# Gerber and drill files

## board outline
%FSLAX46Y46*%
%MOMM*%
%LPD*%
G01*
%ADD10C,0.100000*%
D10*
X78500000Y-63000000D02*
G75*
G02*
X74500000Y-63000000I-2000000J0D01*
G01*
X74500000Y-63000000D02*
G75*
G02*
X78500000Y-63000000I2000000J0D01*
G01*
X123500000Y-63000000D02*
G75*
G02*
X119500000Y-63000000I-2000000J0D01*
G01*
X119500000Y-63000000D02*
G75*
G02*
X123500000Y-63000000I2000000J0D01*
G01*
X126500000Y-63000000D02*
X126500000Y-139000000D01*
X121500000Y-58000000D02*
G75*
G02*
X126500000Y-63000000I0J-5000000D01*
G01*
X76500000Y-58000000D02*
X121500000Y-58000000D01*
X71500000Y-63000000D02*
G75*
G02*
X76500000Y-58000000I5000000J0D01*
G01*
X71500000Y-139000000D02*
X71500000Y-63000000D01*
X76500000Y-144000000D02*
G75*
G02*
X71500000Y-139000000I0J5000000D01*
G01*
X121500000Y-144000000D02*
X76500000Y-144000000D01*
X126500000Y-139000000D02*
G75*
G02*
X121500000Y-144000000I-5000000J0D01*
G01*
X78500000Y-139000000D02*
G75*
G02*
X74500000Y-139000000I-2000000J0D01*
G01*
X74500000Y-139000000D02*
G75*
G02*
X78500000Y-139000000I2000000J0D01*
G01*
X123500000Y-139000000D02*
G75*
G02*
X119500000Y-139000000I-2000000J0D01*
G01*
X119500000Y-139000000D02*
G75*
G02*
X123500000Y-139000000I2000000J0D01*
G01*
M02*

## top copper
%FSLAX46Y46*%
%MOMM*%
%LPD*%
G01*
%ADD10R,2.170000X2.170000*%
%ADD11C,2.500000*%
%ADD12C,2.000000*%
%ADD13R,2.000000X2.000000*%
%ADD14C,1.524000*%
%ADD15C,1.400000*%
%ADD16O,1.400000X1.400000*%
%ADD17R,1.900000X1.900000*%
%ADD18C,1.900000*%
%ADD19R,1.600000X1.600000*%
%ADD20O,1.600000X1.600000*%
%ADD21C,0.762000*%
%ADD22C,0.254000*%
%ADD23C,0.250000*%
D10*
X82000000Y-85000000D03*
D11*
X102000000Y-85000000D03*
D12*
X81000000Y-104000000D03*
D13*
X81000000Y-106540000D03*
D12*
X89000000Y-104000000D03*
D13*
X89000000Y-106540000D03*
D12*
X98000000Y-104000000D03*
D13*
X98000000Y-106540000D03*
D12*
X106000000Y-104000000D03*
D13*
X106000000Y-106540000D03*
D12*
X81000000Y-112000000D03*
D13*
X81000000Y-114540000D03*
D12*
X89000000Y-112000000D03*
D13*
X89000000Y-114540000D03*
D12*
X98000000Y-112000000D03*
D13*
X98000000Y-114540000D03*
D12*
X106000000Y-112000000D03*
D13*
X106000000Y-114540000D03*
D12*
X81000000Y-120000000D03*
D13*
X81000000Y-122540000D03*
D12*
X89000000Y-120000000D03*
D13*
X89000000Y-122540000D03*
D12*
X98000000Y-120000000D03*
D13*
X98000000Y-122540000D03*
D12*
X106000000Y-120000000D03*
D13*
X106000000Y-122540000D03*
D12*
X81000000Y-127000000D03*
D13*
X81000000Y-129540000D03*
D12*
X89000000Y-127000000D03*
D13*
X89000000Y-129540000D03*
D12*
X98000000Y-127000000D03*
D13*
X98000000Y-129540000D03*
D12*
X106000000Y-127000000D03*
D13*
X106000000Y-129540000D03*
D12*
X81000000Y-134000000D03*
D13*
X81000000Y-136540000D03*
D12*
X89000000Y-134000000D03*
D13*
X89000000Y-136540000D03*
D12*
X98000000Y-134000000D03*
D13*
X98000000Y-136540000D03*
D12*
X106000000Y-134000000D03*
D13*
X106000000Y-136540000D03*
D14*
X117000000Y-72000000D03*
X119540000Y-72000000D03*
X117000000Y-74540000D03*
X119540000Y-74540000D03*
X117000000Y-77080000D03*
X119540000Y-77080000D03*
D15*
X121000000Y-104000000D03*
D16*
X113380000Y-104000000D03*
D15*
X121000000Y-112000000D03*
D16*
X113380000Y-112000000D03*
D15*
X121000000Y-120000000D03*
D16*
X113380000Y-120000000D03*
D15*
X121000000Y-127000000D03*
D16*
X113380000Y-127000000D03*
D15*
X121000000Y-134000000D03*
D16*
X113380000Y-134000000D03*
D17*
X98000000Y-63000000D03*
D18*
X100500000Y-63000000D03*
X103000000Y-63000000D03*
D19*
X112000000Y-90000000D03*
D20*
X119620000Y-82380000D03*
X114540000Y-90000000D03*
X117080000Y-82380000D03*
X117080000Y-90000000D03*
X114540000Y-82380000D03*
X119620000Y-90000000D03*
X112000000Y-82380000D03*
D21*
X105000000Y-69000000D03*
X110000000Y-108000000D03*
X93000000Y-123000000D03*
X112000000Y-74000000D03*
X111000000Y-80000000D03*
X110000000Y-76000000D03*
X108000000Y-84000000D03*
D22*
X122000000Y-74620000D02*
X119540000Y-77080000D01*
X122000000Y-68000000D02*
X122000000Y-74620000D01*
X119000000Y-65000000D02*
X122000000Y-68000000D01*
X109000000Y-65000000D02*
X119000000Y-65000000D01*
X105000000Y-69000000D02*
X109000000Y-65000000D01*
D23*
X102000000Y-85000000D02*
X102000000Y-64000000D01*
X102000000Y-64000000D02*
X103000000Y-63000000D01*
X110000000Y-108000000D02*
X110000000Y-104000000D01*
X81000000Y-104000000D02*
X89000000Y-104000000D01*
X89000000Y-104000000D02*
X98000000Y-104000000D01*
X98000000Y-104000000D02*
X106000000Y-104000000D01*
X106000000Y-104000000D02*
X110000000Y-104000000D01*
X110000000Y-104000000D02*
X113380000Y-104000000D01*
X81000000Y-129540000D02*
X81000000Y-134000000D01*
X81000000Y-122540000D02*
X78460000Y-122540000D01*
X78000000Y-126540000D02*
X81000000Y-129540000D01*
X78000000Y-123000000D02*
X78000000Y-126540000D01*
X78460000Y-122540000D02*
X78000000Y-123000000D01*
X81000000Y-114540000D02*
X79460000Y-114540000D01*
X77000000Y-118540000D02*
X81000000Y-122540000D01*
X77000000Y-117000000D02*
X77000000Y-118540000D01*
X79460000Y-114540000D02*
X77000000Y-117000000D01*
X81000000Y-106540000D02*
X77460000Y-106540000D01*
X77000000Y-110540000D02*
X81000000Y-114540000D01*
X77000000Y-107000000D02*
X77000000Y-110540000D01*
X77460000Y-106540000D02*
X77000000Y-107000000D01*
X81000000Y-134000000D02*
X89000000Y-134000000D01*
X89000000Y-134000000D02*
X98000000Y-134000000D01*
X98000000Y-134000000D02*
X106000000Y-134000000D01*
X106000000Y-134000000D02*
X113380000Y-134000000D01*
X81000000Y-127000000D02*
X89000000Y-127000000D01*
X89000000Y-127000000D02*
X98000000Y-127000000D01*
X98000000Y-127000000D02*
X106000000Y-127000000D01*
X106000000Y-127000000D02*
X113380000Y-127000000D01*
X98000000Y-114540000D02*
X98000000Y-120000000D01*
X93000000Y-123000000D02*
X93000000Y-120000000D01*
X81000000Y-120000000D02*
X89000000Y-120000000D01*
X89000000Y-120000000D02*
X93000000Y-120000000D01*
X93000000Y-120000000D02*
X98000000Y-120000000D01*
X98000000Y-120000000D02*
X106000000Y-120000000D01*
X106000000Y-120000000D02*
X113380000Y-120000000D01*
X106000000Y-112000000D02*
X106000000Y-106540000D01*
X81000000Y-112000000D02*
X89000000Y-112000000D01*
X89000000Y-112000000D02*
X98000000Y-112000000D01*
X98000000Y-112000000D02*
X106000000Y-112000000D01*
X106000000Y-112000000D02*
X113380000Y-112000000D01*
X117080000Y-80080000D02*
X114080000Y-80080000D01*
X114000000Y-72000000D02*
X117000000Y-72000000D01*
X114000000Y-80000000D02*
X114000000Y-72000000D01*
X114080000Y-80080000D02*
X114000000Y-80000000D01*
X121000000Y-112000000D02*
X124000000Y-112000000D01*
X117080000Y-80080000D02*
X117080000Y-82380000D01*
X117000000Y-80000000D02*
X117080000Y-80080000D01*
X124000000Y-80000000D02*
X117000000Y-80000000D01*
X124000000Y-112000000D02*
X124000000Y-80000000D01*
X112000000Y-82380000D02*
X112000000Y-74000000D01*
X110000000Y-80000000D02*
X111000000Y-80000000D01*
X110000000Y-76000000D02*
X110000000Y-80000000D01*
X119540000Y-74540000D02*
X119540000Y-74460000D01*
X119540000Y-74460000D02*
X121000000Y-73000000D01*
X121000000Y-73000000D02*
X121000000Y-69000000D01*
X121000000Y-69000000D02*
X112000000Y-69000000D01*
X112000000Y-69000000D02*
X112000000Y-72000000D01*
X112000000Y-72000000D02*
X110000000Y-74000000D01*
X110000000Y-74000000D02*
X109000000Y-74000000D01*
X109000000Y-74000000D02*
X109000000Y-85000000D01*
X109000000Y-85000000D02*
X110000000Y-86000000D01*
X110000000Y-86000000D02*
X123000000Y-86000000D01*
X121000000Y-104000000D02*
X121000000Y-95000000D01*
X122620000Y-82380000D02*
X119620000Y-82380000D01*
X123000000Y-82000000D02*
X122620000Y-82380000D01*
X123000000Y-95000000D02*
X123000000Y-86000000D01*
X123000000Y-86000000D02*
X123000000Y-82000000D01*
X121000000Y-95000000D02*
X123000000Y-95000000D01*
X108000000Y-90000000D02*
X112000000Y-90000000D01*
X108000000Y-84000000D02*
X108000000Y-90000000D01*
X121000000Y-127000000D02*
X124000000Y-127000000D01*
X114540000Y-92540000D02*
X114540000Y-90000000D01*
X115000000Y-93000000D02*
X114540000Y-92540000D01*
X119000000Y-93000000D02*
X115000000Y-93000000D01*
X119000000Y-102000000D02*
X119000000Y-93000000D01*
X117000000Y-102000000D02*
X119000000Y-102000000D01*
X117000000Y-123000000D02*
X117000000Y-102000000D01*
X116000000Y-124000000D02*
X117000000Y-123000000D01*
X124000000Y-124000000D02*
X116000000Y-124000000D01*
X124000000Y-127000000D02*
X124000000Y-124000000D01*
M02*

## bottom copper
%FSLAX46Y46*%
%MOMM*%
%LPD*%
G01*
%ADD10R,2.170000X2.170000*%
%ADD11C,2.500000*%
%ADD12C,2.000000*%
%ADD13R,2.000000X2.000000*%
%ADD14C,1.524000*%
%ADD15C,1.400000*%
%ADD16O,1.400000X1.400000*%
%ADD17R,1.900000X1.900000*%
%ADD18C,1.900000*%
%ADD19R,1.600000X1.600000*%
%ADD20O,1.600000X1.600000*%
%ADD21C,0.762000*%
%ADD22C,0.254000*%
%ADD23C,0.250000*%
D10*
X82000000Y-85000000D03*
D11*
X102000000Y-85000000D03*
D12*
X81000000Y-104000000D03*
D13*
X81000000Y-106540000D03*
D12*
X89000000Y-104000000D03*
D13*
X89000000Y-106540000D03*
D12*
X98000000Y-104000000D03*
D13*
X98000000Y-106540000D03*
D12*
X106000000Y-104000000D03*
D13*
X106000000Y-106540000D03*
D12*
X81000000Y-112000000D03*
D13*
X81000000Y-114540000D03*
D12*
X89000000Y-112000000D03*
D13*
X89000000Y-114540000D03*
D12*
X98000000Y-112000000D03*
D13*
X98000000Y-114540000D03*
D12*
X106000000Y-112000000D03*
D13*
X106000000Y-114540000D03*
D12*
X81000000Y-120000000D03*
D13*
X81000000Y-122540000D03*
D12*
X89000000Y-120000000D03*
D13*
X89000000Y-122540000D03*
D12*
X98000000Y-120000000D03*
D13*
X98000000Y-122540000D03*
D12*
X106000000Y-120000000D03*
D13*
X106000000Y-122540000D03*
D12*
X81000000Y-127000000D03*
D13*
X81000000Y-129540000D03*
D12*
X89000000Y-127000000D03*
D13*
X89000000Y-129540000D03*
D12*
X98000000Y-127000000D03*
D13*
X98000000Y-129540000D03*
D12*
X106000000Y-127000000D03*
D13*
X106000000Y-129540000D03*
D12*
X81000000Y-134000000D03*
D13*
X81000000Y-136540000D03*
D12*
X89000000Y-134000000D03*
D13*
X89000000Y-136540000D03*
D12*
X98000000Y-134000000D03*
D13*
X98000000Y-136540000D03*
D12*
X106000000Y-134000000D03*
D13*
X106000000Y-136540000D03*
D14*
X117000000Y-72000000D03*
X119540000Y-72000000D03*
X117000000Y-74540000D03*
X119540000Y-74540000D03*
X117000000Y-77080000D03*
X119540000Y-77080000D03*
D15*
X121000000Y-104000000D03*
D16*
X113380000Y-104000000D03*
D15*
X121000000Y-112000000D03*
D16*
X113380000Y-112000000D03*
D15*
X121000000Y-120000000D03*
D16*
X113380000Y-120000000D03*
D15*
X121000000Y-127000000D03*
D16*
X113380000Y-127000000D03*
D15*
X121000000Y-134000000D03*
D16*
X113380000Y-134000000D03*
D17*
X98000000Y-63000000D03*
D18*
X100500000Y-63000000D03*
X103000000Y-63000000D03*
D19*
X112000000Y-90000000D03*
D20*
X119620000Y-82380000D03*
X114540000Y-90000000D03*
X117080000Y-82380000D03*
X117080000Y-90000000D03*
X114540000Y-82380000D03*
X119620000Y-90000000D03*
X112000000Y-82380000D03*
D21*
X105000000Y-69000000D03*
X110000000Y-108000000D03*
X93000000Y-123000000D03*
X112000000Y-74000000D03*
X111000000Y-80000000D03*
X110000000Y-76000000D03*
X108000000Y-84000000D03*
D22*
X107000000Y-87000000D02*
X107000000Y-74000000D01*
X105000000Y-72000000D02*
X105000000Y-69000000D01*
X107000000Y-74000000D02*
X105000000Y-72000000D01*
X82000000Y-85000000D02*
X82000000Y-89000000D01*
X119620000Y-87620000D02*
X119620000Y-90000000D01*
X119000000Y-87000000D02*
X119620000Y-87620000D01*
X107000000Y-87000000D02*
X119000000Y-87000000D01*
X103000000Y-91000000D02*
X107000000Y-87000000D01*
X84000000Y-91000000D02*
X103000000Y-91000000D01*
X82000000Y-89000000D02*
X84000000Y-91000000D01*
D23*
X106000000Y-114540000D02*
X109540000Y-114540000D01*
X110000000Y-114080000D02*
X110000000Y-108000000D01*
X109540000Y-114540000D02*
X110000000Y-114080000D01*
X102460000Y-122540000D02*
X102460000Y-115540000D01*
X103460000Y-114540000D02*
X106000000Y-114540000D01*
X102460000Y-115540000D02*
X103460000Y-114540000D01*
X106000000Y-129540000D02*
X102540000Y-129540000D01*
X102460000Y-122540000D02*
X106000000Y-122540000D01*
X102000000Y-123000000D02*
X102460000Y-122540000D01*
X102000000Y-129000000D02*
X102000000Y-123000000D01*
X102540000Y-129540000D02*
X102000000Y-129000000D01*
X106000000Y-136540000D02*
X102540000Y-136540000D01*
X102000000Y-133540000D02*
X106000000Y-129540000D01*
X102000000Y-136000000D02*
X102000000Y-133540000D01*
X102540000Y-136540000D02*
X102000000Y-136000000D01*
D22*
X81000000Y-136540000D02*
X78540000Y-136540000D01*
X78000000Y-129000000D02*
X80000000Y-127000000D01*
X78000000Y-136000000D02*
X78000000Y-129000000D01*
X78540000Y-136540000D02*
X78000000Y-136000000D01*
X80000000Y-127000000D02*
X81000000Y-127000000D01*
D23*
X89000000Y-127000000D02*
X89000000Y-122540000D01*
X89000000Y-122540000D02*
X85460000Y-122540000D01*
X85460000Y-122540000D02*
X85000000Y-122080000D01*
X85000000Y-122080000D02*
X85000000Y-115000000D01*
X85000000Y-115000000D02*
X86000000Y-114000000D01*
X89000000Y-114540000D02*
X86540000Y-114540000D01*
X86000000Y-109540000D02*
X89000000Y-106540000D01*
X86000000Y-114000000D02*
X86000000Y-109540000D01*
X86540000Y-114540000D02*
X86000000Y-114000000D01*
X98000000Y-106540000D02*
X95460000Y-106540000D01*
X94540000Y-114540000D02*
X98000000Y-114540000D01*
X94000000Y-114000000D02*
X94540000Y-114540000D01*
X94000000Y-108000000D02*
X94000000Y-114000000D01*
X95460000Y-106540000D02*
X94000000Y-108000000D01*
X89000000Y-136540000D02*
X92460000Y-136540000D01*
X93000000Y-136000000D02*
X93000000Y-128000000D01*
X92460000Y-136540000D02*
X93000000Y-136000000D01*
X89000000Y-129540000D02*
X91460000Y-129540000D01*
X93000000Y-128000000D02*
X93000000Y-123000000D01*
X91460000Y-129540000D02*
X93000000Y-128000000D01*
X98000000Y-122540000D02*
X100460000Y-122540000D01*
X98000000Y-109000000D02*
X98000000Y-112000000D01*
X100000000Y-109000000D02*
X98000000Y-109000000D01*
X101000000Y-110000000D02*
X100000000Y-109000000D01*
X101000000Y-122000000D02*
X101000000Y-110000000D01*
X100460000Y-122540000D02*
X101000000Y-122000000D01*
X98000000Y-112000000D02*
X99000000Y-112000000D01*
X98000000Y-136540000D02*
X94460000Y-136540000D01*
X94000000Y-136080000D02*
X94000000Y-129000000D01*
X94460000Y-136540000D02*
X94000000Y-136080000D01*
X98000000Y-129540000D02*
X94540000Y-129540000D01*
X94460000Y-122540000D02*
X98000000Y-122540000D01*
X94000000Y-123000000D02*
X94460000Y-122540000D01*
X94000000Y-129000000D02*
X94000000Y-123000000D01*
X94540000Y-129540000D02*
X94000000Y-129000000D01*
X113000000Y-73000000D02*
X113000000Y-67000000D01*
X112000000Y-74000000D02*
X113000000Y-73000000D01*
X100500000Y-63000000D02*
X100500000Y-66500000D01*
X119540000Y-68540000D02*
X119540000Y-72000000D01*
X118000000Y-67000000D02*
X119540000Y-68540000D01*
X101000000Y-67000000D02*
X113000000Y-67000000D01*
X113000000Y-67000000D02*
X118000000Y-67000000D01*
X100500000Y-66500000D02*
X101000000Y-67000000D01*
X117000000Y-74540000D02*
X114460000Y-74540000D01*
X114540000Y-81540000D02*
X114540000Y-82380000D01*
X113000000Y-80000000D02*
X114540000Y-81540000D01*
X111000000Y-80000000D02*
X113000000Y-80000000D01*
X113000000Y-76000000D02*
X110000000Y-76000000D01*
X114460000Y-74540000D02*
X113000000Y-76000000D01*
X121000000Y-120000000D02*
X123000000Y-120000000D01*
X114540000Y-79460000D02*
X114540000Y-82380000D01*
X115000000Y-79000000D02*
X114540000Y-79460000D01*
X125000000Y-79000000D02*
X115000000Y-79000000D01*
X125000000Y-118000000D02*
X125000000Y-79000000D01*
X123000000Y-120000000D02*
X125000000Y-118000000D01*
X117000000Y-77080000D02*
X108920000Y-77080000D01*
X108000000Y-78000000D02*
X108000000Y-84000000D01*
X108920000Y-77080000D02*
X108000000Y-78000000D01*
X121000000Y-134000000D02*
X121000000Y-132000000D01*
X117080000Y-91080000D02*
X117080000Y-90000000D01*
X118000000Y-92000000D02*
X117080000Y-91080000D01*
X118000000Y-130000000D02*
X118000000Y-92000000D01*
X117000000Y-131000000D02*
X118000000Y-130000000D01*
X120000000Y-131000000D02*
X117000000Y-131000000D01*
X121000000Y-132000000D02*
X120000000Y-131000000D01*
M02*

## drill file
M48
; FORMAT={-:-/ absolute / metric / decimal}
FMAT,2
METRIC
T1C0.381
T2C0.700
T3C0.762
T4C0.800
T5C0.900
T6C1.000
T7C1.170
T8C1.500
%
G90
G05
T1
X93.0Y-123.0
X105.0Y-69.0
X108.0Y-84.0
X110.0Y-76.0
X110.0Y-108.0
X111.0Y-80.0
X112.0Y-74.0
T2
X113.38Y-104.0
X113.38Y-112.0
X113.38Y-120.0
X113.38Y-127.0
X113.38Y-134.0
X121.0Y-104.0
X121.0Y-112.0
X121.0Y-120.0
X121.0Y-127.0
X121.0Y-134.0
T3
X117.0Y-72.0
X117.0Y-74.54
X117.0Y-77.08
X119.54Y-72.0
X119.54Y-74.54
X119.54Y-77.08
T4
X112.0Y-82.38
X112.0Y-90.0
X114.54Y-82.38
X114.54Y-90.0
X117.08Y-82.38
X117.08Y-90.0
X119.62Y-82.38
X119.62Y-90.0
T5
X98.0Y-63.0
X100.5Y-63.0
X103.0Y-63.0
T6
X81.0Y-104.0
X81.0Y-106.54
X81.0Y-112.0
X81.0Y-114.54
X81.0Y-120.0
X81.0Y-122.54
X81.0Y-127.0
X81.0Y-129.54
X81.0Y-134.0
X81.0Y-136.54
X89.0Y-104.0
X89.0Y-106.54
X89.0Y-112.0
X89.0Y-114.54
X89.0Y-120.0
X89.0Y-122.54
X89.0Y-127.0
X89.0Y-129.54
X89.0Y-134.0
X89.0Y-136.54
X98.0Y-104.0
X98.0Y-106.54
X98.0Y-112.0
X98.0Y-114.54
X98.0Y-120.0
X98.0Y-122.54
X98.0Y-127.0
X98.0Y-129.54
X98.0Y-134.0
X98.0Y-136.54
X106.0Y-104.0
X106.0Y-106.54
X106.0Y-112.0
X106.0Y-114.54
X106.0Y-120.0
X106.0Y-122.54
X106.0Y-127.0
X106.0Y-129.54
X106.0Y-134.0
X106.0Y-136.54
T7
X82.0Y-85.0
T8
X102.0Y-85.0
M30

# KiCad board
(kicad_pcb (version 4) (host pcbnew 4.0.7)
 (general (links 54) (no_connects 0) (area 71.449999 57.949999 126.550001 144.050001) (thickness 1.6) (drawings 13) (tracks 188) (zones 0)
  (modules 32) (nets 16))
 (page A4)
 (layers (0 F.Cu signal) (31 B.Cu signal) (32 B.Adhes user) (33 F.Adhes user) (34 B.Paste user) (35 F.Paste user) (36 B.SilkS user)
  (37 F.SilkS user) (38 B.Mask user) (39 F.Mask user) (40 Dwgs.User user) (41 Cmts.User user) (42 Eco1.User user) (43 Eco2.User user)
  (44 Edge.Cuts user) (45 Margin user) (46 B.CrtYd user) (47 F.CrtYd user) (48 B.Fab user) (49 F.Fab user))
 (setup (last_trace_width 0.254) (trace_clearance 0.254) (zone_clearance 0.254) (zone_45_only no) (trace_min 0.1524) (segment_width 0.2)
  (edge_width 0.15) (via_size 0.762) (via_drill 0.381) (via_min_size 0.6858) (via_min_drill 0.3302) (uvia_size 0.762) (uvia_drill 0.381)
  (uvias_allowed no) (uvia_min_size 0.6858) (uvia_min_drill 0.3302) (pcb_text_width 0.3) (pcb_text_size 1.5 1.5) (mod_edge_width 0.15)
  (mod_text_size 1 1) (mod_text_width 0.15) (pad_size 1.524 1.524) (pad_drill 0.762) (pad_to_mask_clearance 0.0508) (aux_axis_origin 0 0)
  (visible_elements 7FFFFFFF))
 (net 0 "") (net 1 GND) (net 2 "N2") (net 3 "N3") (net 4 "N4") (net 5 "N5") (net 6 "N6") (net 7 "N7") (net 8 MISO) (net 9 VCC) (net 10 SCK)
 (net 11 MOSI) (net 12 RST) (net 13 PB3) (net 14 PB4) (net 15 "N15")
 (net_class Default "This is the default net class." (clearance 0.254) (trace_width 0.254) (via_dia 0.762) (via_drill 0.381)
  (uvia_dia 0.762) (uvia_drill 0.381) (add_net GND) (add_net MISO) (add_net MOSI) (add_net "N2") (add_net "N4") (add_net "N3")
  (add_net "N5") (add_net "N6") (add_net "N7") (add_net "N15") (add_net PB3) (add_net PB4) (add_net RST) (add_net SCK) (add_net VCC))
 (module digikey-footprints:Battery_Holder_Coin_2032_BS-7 (layer F.Cu) (at 82 85)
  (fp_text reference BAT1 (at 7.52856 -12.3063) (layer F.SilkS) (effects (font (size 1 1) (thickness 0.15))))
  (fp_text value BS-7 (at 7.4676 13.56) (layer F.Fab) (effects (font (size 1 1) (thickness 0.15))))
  (pad Neg thru_hole rect (at 0 0) (size 2.17 2.17) (drill 1.17) (layers *.Cu *.Mask) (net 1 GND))
  (pad Pos thru_hole circle (at 20 0) (size 2.5 2.5) (drill 1.5) (layers *.Cu *.Mask) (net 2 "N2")))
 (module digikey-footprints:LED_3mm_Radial (layer F.Cu) (at 81 104 90)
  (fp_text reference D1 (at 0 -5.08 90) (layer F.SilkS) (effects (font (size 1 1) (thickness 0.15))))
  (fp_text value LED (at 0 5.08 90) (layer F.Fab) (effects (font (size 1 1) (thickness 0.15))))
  (pad 2 thru_hole circle (at 0 0 90) (size 2 2) (drill 1) (layers *.Cu *.Mask) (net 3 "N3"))
  (pad 1 thru_hole rect (at -2.54 0 90) (size 2 2) (drill 1) (layers *.Cu *.Mask) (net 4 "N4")))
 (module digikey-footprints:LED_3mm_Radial (layer F.Cu) (at 89 104 90)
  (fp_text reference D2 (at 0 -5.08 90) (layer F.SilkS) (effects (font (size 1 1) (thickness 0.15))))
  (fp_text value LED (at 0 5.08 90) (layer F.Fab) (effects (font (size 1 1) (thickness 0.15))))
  (pad 2 thru_hole circle (at 0 0 90) (size 2 2) (drill 1) (layers *.Cu *.Mask) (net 3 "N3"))
  (pad 1 thru_hole rect (at -2.54 0 90) (size 2 2) (drill 1) (layers *.Cu *.Mask) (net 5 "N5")))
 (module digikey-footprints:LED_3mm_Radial (layer F.Cu) (at 98 104 90)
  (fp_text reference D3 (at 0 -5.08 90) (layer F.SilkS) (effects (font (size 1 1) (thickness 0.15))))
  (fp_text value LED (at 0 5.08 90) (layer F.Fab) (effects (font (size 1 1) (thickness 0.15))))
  (pad 2 thru_hole circle (at 0 0 90) (size 2 2) (drill 1) (layers *.Cu *.Mask) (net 3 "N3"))
  (pad 1 thru_hole rect (at -2.54 0 90) (size 2 2) (drill 1) (layers *.Cu *.Mask) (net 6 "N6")))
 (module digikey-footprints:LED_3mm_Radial (layer F.Cu) (at 106 104 90)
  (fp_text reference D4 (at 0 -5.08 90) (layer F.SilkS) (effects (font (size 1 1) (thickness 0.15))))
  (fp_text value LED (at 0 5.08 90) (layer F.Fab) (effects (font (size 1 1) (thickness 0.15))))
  (pad 2 thru_hole circle (at 0 0 90) (size 2 2) (drill 1) (layers *.Cu *.Mask) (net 3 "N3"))
  (pad 1 thru_hole rect (at -2.54 0 90) (size 2 2) (drill 1) (layers *.Cu *.Mask) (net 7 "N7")))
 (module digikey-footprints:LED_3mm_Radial (layer F.Cu) (at 81 112 90)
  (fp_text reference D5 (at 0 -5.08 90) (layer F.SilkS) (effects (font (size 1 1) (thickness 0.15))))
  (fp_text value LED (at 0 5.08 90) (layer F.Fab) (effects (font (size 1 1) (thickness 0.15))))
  (pad 2 thru_hole circle (at 0 0 90) (size 2 2) (drill 1) (layers *.Cu *.Mask) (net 7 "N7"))
  (pad 1 thru_hole rect (at -2.54 0 90) (size 2 2) (drill 1) (layers *.Cu *.Mask) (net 4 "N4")))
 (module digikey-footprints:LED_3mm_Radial (layer F.Cu) (at 89 112 90)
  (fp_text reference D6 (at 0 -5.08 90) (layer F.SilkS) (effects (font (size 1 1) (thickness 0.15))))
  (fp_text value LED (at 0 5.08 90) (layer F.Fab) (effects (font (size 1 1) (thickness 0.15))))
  (pad 2 thru_hole circle (at 0 0 90) (size 2 2) (drill 1) (layers *.Cu *.Mask) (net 7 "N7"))
  (pad 1 thru_hole rect (at -2.54 0 90) (size 2 2) (drill 1) (layers *.Cu *.Mask) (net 5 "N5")))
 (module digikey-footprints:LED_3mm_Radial (layer F.Cu) (at 98 112 90)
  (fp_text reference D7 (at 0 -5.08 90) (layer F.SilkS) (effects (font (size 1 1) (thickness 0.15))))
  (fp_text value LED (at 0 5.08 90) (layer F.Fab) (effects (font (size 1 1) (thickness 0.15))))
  (pad 2 thru_hole circle (at 0 0 90) (size 2 2) (drill 1) (layers *.Cu *.Mask) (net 7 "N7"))
  (pad 1 thru_hole rect (at -2.54 0 90) (size 2 2) (drill 1) (layers *.Cu *.Mask) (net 6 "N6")))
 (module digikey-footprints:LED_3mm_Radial (layer F.Cu) (at 106 112 90)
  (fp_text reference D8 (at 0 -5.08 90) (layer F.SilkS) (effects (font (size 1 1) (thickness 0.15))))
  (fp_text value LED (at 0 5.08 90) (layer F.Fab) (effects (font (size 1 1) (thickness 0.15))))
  (pad 2 thru_hole circle (at 0 0 90) (size 2 2) (drill 1) (layers *.Cu *.Mask) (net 7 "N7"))
  (pad 1 thru_hole rect (at -2.54 0 90) (size 2 2) (drill 1) (layers *.Cu *.Mask) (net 3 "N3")))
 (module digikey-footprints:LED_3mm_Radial (layer F.Cu) (at 81 120 90)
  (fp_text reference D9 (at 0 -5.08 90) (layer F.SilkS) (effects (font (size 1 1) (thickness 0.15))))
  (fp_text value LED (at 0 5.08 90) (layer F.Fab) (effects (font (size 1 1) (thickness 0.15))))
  (pad 2 thru_hole circle (at 0 0 90) (size 2 2) (drill 1) (layers *.Cu *.Mask) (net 6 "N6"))
  (pad 1 thru_hole rect (at -2.54 0 90) (size 2 2) (drill 1) (layers *.Cu *.Mask) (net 4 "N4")))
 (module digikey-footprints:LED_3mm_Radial (layer F.Cu) (at 89 120 90)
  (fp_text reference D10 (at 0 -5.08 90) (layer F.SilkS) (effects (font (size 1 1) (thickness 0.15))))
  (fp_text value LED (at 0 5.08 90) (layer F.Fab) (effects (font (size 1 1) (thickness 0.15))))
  (pad 2 thru_hole circle (at 0 0 90) (size 2 2) (drill 1) (layers *.Cu *.Mask) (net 6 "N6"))
  (pad 1 thru_hole rect (at -2.54 0 90) (size 2 2) (drill 1) (layers *.Cu *.Mask) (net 5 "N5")))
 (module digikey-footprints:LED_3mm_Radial (layer F.Cu) (at 98 120 90)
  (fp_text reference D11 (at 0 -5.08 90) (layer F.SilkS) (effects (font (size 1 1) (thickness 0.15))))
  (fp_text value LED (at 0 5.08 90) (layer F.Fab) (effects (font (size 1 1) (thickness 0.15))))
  (pad 2 thru_hole circle (at 0 0 90) (size 2 2) (drill 1) (layers *.Cu *.Mask) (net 6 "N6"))
  (pad 1 thru_hole rect (at -2.54 0 90) (size 2 2) (drill 1) (layers *.Cu *.Mask) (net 7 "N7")))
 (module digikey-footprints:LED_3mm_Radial (layer F.Cu) (at 106 120 90)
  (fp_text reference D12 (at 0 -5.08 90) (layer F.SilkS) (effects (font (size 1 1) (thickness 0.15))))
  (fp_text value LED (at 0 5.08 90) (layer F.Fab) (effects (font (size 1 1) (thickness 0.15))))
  (pad 2 thru_hole circle (at 0 0 90) (size 2 2) (drill 1) (layers *.Cu *.Mask) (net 6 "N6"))
  (pad 1 thru_hole rect (at -2.54 0 90) (size 2 2) (drill 1) (layers *.Cu *.Mask) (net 3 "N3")))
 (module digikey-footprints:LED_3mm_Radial (layer F.Cu) (at 81 127 90)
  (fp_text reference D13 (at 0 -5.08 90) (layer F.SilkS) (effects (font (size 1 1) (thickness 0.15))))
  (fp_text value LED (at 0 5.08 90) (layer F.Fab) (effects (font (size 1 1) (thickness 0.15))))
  (pad 2 thru_hole circle (at 0 0 90) (size 2 2) (drill 1) (layers *.Cu *.Mask) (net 5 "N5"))
  (pad 1 thru_hole rect (at -2.54 0 90) (size 2 2) (drill 1) (layers *.Cu *.Mask) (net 4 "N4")))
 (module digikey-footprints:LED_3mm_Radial (layer F.Cu) (at 89 127 90)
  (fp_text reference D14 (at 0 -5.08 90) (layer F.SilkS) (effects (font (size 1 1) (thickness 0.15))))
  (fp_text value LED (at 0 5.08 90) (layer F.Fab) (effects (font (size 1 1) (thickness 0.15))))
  (pad 2 thru_hole circle (at 0 0 90) (size 2 2) (drill 1) (layers *.Cu *.Mask) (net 5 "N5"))
  (pad 1 thru_hole rect (at -2.54 0 90) (size 2 2) (drill 1) (layers *.Cu *.Mask) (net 6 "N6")))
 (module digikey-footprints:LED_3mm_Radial (layer F.Cu) (at 98 127 90)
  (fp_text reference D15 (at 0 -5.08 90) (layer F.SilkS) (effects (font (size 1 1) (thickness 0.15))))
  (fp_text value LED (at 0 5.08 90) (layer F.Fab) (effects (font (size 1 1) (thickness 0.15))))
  (pad 2 thru_hole circle (at 0 0 90) (size 2 2) (drill 1) (layers *.Cu *.Mask) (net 5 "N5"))
  (pad 1 thru_hole rect (at -2.54 0 90) (size 2 2) (drill 1) (layers *.Cu *.Mask) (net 7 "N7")))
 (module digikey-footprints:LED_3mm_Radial (layer F.Cu) (at 106 127 90)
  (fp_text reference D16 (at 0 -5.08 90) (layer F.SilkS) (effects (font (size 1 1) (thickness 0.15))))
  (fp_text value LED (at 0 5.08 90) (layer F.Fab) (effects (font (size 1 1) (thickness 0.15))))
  (pad 2 thru_hole circle (at 0 0 90) (size 2 2) (drill 1) (layers *.Cu *.Mask) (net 5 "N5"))
  (pad 1 thru_hole rect (at -2.54 0 90) (size 2 2) (drill 1) (layers *.Cu *.Mask) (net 3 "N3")))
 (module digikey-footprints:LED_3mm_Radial (layer F.Cu) (at 81 134 90)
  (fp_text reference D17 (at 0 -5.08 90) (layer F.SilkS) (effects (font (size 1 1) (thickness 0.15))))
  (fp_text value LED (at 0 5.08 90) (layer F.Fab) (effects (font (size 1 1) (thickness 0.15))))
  (pad 2 thru_hole circle (at 0 0 90) (size 2 2) (drill 1) (layers *.Cu *.Mask) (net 4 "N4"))
  (pad 1 thru_hole rect (at -2.54 0 90) (size 2 2) (drill 1) (layers *.Cu *.Mask) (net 5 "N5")))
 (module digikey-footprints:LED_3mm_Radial (layer F.Cu) (at 89 134 90)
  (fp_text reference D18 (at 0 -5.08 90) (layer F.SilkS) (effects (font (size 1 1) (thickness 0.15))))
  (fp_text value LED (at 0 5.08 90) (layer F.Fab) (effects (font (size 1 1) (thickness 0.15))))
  (pad 2 thru_hole circle (at 0 0 90) (size 2 2) (drill 1) (layers *.Cu *.Mask) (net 4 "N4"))
  (pad 1 thru_hole rect (at -2.54 0 90) (size 2 2) (drill 1) (layers *.Cu *.Mask) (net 6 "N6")))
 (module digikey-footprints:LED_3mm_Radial (layer F.Cu) (at 98 134 90)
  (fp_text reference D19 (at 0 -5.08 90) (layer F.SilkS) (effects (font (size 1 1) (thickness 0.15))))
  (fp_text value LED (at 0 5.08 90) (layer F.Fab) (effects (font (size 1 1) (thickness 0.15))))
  (pad 2 thru_hole circle (at 0 0 90) (size 2 2) (drill 1) (layers *.Cu *.Mask) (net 4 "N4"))
  (pad 1 thru_hole rect (at -2.54 0 90) (size 2 2) (drill 1) (layers *.Cu *.Mask) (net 7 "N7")))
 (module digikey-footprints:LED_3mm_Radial (layer F.Cu) (at 106 134 90)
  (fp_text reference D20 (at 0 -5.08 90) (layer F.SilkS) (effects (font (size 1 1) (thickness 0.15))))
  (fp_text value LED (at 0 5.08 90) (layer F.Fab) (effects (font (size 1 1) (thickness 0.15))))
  (pad 2 thru_hole circle (at 0 0 90) (size 2 2) (drill 1) (layers *.Cu *.Mask) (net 4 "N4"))
  (pad 1 thru_hole rect (at -2.54 0 90) (size 2 2) (drill 1) (layers *.Cu *.Mask) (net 3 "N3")))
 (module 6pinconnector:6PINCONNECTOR (layer F.Cu) (at 117 72 270)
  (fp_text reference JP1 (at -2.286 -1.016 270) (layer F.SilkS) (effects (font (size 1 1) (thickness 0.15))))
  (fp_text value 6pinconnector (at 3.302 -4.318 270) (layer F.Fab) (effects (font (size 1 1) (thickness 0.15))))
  (pad 1 thru_hole circle (at 0 0 270) (size 1.524 1.524) (drill 0.762) (layers *.Cu *.Mask) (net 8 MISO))
  (pad 2 thru_hole circle (at 0 -2.54 270) (size 1.524 1.524) (drill 0.762) (layers *.Cu *.Mask) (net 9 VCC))
  (pad 3 thru_hole circle (at 2.54 0 270) (size 1.524 1.524) (drill 0.762) (layers *.Cu *.Mask) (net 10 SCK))
  (pad 4 thru_hole circle (at 2.54 -2.54 270) (size 1.524 1.524) (drill 0.762) (layers *.Cu *.Mask) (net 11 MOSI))
  (pad 5 thru_hole circle (at 5.08 0 270) (size 1.524 1.524) (drill 0.762) (layers *.Cu *.Mask) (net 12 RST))
  (pad 6 thru_hole circle (at 5.08 -2.54 270) (size 1.524 1.524) (drill 0.762) (layers *.Cu *.Mask) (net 1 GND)))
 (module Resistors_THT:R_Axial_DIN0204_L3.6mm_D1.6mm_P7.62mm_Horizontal (layer F.Cu) (at 121 104 180)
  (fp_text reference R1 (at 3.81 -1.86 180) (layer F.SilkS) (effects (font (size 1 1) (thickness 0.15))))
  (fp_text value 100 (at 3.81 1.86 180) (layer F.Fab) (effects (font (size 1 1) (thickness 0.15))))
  (pad 1 thru_hole circle (at 0 0 180) (size 1.4 1.4) (drill 0.7) (layers *.Cu *.Mask) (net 11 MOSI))
  (pad 2 thru_hole oval (at 7.62 0 180) (size 1.4 1.4) (drill 0.7) (layers *.Cu *.Mask) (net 3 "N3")))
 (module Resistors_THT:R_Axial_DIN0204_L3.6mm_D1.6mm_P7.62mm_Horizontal (layer F.Cu) (at 121 112 180)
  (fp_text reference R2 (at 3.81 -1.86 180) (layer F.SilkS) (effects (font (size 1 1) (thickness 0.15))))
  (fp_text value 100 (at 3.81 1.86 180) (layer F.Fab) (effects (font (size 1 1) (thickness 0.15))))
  (pad 1 thru_hole circle (at 0 0 180) (size 1.4 1.4) (drill 0.7) (layers *.Cu *.Mask) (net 8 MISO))
  (pad 2 thru_hole oval (at 7.62 0 180) (size 1.4 1.4) (drill 0.7) (layers *.Cu *.Mask) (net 7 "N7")))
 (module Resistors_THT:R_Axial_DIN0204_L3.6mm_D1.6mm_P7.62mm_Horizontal (layer F.Cu) (at 121 120 180)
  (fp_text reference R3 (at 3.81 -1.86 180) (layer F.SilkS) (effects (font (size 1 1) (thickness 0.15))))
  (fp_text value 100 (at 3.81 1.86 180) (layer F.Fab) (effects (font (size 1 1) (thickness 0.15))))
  (pad 1 thru_hole circle (at 0 0 180) (size 1.4 1.4) (drill 0.7) (layers *.Cu *.Mask) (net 10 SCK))
  (pad 2 thru_hole oval (at 7.62 0 180) (size 1.4 1.4) (drill 0.7) (layers *.Cu *.Mask) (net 6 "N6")))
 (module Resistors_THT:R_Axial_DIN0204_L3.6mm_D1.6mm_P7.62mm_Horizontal (layer F.Cu) (at 121 127 180)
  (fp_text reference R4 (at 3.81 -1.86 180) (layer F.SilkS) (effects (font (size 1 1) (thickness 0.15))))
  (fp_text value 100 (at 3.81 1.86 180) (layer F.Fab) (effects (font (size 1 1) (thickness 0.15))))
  (pad 1 thru_hole circle (at 0 0 180) (size 1.4 1.4) (drill 0.7) (layers *.Cu *.Mask) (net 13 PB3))
  (pad 2 thru_hole oval (at 7.62 0 180) (size 1.4 1.4) (drill 0.7) (layers *.Cu *.Mask) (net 5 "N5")))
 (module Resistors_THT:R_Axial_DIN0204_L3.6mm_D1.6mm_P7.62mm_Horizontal (layer F.Cu) (at 121 134 180)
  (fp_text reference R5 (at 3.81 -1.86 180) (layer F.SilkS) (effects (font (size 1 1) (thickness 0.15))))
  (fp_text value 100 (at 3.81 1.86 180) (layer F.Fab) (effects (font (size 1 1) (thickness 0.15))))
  (pad 1 thru_hole circle (at 0 0 180) (size 1.4 1.4) (drill 0.7) (layers *.Cu *.Mask) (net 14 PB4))
  (pad 2 thru_hole oval (at 7.62 0 180) (size 1.4 1.4) (drill 0.7) (layers *.Cu *.Mask) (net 4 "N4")))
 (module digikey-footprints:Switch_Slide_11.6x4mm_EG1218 (layer F.Cu) (at 98 63)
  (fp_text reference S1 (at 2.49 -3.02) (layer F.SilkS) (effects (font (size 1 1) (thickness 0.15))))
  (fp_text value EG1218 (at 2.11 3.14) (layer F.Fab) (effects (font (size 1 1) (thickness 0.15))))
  (pad 1 thru_hole rect (at 0 0) (size 1.9 1.9) (drill 0.9) (layers *.Cu *.Mask) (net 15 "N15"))
  (pad 2 thru_hole circle (at 2.5 0) (size 1.9 1.9) (drill 0.9) (layers *.Cu *.Mask) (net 9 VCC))
  (pad 3 thru_hole circle (at 5 0) (size 1.9 1.9) (drill 0.9) (layers *.Cu *.Mask) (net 2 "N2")))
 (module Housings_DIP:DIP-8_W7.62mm (layer F.Cu) (at 112 90 90)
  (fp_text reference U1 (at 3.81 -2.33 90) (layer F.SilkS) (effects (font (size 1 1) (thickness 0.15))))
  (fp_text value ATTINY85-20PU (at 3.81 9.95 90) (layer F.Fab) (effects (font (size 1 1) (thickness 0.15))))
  (pad 1 thru_hole rect (at 0 0 90) (size 1.6 1.6) (drill 0.8) (layers *.Cu *.Mask) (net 12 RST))
  (pad 5 thru_hole oval (at 7.62 7.62 90) (size 1.6 1.6) (drill 0.8) (layers *.Cu *.Mask) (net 11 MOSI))
  (pad 2 thru_hole oval (at 0 2.54 90) (size 1.6 1.6) (drill 0.8) (layers *.Cu *.Mask) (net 13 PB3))
  (pad 6 thru_hole oval (at 7.62 5.08 90) (size 1.6 1.6) (drill 0.8) (layers *.Cu *.Mask) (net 8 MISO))
  (pad 3 thru_hole oval (at 0 5.08 90) (size 1.6 1.6) (drill 0.8) (layers *.Cu *.Mask) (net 14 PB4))
  (pad 7 thru_hole oval (at 7.62 2.54 90) (size 1.6 1.6) (drill 0.8) (layers *.Cu *.Mask) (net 10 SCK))
  (pad 4 thru_hole oval (at 0 7.62 90) (size 1.6 1.6) (drill 0.8) (layers *.Cu *.Mask) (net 1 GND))
  (pad 8 thru_hole oval (at 7.62 0 90) (size 1.6 1.6) (drill 0.8) (layers *.Cu *.Mask) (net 9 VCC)))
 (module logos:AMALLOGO (layer F.Cu) (at 85 64)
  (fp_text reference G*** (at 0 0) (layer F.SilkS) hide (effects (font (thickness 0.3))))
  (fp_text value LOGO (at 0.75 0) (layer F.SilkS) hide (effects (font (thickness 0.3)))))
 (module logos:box (layer F.Cu) (at 98 99)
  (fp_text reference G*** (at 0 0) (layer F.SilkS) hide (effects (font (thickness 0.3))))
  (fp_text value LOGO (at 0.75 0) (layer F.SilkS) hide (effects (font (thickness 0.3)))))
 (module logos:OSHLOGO (layer F.Cu) (at 109 70)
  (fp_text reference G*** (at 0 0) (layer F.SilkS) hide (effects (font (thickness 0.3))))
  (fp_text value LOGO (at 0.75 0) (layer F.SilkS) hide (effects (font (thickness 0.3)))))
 (gr_circle (center 76.5 63) (end 78.5 63) (layer Edge.Cuts) (width 0.1))
 (gr_circle (center 121.5 63) (end 123.5 63) (layer Edge.Cuts) (width 0.1))
 (gr_line (start 126.5 63) (end 126.5 139) (layer Edge.Cuts) (width 0.1))
 (gr_arc (start 121.5 63) (end 126.5 63) (angle -90) (layer Edge.Cuts) (width 0.1))
 (gr_line (start 76.5 58) (end 121.5 58) (layer Edge.Cuts) (width 0.1))
 (gr_arc (start 76.5 63) (end 76.5 58) (angle -90) (layer Edge.Cuts) (width 0.1))
 (gr_line (start 71.5 139) (end 71.5 63) (layer Edge.Cuts) (width 0.1))
 (gr_arc (start 76.5 139) (end 71.5 139) (angle -90) (layer Edge.Cuts) (width 0.1))
 (gr_line (start 121.5 144) (end 76.5 144) (layer Edge.Cuts) (width 0.1))
 (gr_arc (start 121.5 139) (end 121.5 144) (angle -90) (layer Edge.Cuts) (width 0.1))
 (gr_circle (center 76.5 139) (end 78.5 139) (layer Edge.Cuts) (width 0.1))
 (gr_circle (center 121.5 139) (end 123.5 139) (layer Edge.Cuts) (width 0.1))
 (segment (start 107 87) (end 107 74) (width 0.254) (layer B.Cu) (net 1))
 (segment (start 122 74.62) (end 119.54 77.08) (width 0.254) (layer F.Cu) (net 1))
 (segment (start 122 68) (end 122 74.62) (width 0.254) (layer F.Cu) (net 1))
 (segment (start 119 65) (end 122 68) (width 0.254) (layer F.Cu) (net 1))
 (segment (start 109 65) (end 119 65) (width 0.254) (layer F.Cu) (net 1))
 (segment (start 105 69) (end 109 65) (width 0.254) (layer F.Cu) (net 1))
 (via (at 105 69) (size 0.762) (drill 0.381) (layers F.Cu B.Cu) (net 1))
 (segment (start 105 72) (end 105 69) (width 0.254) (layer B.Cu) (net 1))
 (segment (start 107 74) (end 105 72) (width 0.254) (layer B.Cu) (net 1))
 (segment (start 82 85) (end 82 89) (width 0.254) (layer B.Cu) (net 1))
 (segment (start 119.62 87.62) (end 119.62 90) (width 0.254) (layer B.Cu) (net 1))
 (segment (start 119 87) (end 119.62 87.62) (width 0.254) (layer B.Cu) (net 1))
 (segment (start 107 87) (end 119 87) (width 0.254) (layer B.Cu) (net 1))
 (segment (start 103 91) (end 107 87) (width 0.254) (layer B.Cu) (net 1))
 (segment (start 84 91) (end 103 91) (width 0.254) (layer B.Cu) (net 1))
 (segment (start 82 89) (end 84 91) (width 0.254) (layer B.Cu) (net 1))
 (segment (start 102 85) (end 102 64) (width 0.25) (layer F.Cu) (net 2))
 (segment (start 102 64) (end 103 63) (width 0.25) (layer F.Cu) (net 2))
 (segment (start 106 114.54) (end 109.54 114.54) (width 0.25) (layer B.Cu) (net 3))
 (segment (start 110 108) (end 110 104) (width 0.25) (layer F.Cu) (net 3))
 (via (at 110 108) (size 0.762) (drill 0.381) (layers F.Cu B.Cu) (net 3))
 (segment (start 110 114.08) (end 110 108) (width 0.25) (layer B.Cu) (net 3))
 (segment (start 109.54 114.54) (end 110 114.08) (width 0.25) (layer B.Cu) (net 3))
 (segment (start 102.46 122.54) (end 102.46 115.54) (width 0.25) (layer B.Cu) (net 3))
 (segment (start 103.46 114.54) (end 106 114.54) (width 0.25) (layer B.Cu) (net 3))
 (segment (start 102.46 115.54) (end 103.46 114.54) (width 0.25) (layer B.Cu) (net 3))
 (segment (start 106 129.54) (end 102.54 129.54) (width 0.25) (layer B.Cu) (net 3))
 (segment (start 102.46 122.54) (end 106 122.54) (width 0.25) (layer B.Cu) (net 3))
 (segment (start 102 123) (end 102.46 122.54) (width 0.25) (layer B.Cu) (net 3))
 (segment (start 102 129) (end 102 123) (width 0.25) (layer B.Cu) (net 3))
 (segment (start 102.54 129.54) (end 102 129) (width 0.25) (layer B.Cu) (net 3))
 (segment (start 106 136.54) (end 102.54 136.54) (width 0.25) (layer B.Cu) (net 3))
 (segment (start 102 133.54) (end 106 129.54) (width 0.25) (layer B.Cu) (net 3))
 (segment (start 102 136) (end 102 133.54) (width 0.25) (layer B.Cu) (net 3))
 (segment (start 102.54 136.54) (end 102 136) (width 0.25) (layer B.Cu) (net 3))
 (segment (start 81 104) (end 89 104) (width 0.25) (layer F.Cu) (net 3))
 (segment (start 89 104) (end 98 104) (width 0.25) (layer F.Cu) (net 3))
 (segment (start 98 104) (end 106 104) (width 0.25) (layer F.Cu) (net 3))
 (segment (start 106 104) (end 110 104) (width 0.25) (layer F.Cu) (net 3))
 (segment (start 110 104) (end 113.38 104) (width 0.25) (layer F.Cu) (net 3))
 (segment (start 81 129.54) (end 81 134) (width 0.25) (layer F.Cu) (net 4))
 (segment (start 81 122.54) (end 78.46 122.54) (width 0.25) (layer F.Cu) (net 4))
 (segment (start 78 126.54) (end 81 129.54) (width 0.25) (layer F.Cu) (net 4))
 (segment (start 78 123) (end 78 126.54) (width 0.25) (layer F.Cu) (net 4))
 (segment (start 78.46 122.54) (end 78 123) (width 0.25) (layer F.Cu) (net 4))
 (segment (start 81 114.54) (end 79.46 114.54) (width 0.25) (layer F.Cu) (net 4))
 (segment (start 77 118.54) (end 81 122.54) (width 0.25) (layer F.Cu) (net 4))
 (segment (start 77 117) (end 77 118.54) (width 0.25) (layer F.Cu) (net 4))
 (segment (start 79.46 114.54) (end 77 117) (width 0.25) (layer F.Cu) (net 4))
 (segment (start 81 106.54) (end 77.46 106.54) (width 0.25) (layer F.Cu) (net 4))
 (segment (start 77 110.54) (end 81 114.54) (width 0.25) (layer F.Cu) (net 4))
 (segment (start 77 107) (end 77 110.54) (width 0.25) (layer F.Cu) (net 4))
 (segment (start 77.46 106.54) (end 77 107) (width 0.25) (layer F.Cu) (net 4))
 (segment (start 81 134) (end 89 134) (width 0.25) (layer F.Cu) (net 4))
 (segment (start 89 134) (end 98 134) (width 0.25) (layer F.Cu) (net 4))
 (segment (start 98 134) (end 106 134) (width 0.25) (layer F.Cu) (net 4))
 (segment (start 106 134) (end 113.38 134) (width 0.25) (layer F.Cu) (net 4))
 (segment (start 81 136.54) (end 78.54 136.54) (width 0.254) (layer B.Cu) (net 5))
 (segment (start 78 129) (end 80 127) (width 0.254) (layer B.Cu) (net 5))
 (segment (start 78 136) (end 78 129) (width 0.254) (layer B.Cu) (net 5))
 (segment (start 78.54 136.54) (end 78 136) (width 0.254) (layer B.Cu) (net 5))
 (segment (start 80 127) (end 81 127) (width 0.254) (layer B.Cu) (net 5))
 (segment (start 89 127) (end 89 122.54) (width 0.25) (layer B.Cu) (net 5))
 (segment (start 89 122.54) (end 85.46 122.54) (width 0.25) (layer B.Cu) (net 5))
 (segment (start 85.46 122.54) (end 85 122.08) (width 0.25) (layer B.Cu) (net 5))
 (segment (start 85 122.08) (end 85 115) (width 0.25) (layer B.Cu) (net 5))
 (segment (start 85 115) (end 86 114) (width 0.25) (layer B.Cu) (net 5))
 (segment (start 89 114.54) (end 86.54 114.54) (width 0.25) (layer B.Cu) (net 5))
 (segment (start 86 109.54) (end 89 106.54) (width 0.25) (layer B.Cu) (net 5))
 (segment (start 86 114) (end 86 109.54) (width 0.25) (layer B.Cu) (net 5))
 (segment (start 86.54 114.54) (end 86 114) (width 0.25) (layer B.Cu) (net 5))
 (segment (start 81 127) (end 89 127) (width 0.25) (layer F.Cu) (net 5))
 (segment (start 89 127) (end 98 127) (width 0.25) (layer F.Cu) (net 5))
 (segment (start 98 127) (end 106 127) (width 0.25) (layer F.Cu) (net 5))
 (segment (start 106 127) (end 113.38 127) (width 0.25) (layer F.Cu) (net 5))
 (segment (start 98 114.54) (end 98 120) (width 0.25) (layer F.Cu) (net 6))
 (segment (start 98 106.54) (end 95.46 106.54) (width 0.25) (layer B.Cu) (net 6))
 (segment (start 94.54 114.54) (end 98 114.54) (width 0.25) (layer B.Cu) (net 6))
 (segment (start 94 114) (end 94.54 114.54) (width 0.25) (layer B.Cu) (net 6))
 (segment (start 94 108) (end 94 114) (width 0.25) (layer B.Cu) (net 6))
 (segment (start 95.46 106.54) (end 94 108) (width 0.25) (layer B.Cu) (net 6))
 (segment (start 89 136.54) (end 92.46 136.54) (width 0.25) (layer B.Cu) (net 6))
 (segment (start 93 136) (end 93 128) (width 0.25) (layer B.Cu) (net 6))
 (segment (start 92.46 136.54) (end 93 136) (width 0.25) (layer B.Cu) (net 6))
 (segment (start 89 129.54) (end 91.46 129.54) (width 0.25) (layer B.Cu) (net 6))
 (segment (start 93 123) (end 93 120) (width 0.25) (layer F.Cu) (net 6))
 (via (at 93 123) (size 0.762) (drill 0.381) (layers F.Cu B.Cu) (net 6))
 (segment (start 93 128) (end 93 123) (width 0.25) (layer B.Cu) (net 6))
 (segment (start 91.46 129.54) (end 93 128) (width 0.25) (layer B.Cu) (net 6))
 (segment (start 81 120) (end 89 120) (width 0.25) (layer F.Cu) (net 6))
 (segment (start 89 120) (end 93 120) (width 0.25) (layer F.Cu) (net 6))
 (segment (start 93 120) (end 98 120) (width 0.25) (layer F.Cu) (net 6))
 (segment (start 98 120) (end 106 120) (width 0.25) (layer F.Cu) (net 6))
 (segment (start 106 120) (end 113.38 120) (width 0.25) (layer F.Cu) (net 6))
 (segment (start 98 122.54) (end 100.46 122.54) (width 0.25) (layer B.Cu) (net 7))
 (segment (start 98 109) (end 98 112) (width 0.25) (layer B.Cu) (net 7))
 (segment (start 100 109) (end 98 109) (width 0.25) (layer B.Cu) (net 7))
 (segment (start 101 110) (end 100 109) (width 0.25) (layer B.Cu) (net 7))
 (segment (start 101 122) (end 101 110) (width 0.25) (layer B.Cu) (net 7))
 (segment (start 100.46 122.54) (end 101 122) (width 0.25) (layer B.Cu) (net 7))
 (segment (start 98 112) (end 99 112) (width 0.25) (layer B.Cu) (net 7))
 (segment (start 106 112) (end 106 106.54) (width 0.25) (layer F.Cu) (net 7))
 (segment (start 98 136.54) (end 94.46 136.54) (width 0.25) (layer B.Cu) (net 7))
 (segment (start 94 136.08) (end 94 129) (width 0.25) (layer B.Cu) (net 7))
 (segment (start 94.46 136.54) (end 94 136.08) (width 0.25) (layer B.Cu) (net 7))
 (segment (start 98 129.54) (end 94.54 129.54) (width 0.25) (layer B.Cu) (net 7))
 (segment (start 94.46 122.54) (end 98 122.54) (width 0.25) (layer B.Cu) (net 7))
 (segment (start 94 123) (end 94.46 122.54) (width 0.25) (layer B.Cu) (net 7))
 (segment (start 94 129) (end 94 123) (width 0.25) (layer B.Cu) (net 7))
 (segment (start 94.54 129.54) (end 94 129) (width 0.25) (layer B.Cu) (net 7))
 (segment (start 81 112) (end 89 112) (width 0.25) (layer F.Cu) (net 7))
 (segment (start 89 112) (end 98 112) (width 0.25) (layer F.Cu) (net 7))
 (segment (start 98 112) (end 106 112) (width 0.25) (layer F.Cu) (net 7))
 (segment (start 106 112) (end 113.38 112) (width 0.25) (layer F.Cu) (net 7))
 (segment (start 117.08 80.08) (end 114.08 80.08) (width 0.25) (layer F.Cu) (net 8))
 (segment (start 114 72) (end 117 72) (width 0.25) (layer F.Cu) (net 8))
 (segment (start 114 80) (end 114 72) (width 0.25) (layer F.Cu) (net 8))
 (segment (start 114.08 80.08) (end 114 80) (width 0.25) (layer F.Cu) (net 8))
 (segment (start 121 112) (end 124 112) (width 0.25) (layer F.Cu) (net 8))
 (segment (start 117.08 80.08) (end 117.08 82.38) (width 0.25) (layer F.Cu) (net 8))
 (segment (start 117 80) (end 117.08 80.08) (width 0.25) (layer F.Cu) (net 8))
 (segment (start 124 80) (end 117 80) (width 0.25) (layer F.Cu) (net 8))
 (segment (start 124 112) (end 124 80) (width 0.25) (layer F.Cu) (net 8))
 (segment (start 112 82.38) (end 112 74) (width 0.25) (layer F.Cu) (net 9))
 (segment (start 113 73) (end 113 67) (width 0.25) (layer B.Cu) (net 9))
 (segment (start 112 74) (end 113 73) (width 0.25) (layer B.Cu) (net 9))
 (via (at 112 74) (size 0.762) (drill 0.381) (layers F.Cu B.Cu) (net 9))
 (segment (start 100.5 63) (end 100.5 66.5) (width 0.25) (layer B.Cu) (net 9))
 (segment (start 119.54 68.54) (end 119.54 72) (width 0.25) (layer B.Cu) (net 9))
 (segment (start 118 67) (end 119.54 68.54) (width 0.25) (layer B.Cu) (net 9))
 (segment (start 101 67) (end 113 67) (width 0.25) (layer B.Cu) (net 9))
 (segment (start 113 67) (end 118 67) (width 0.25) (layer B.Cu) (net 9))
 (segment (start 100.5 66.5) (end 101 67) (width 0.25) (layer B.Cu) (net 9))
 (segment (start 117 74.54) (end 114.46 74.54) (width 0.25) (layer B.Cu) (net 10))
 (segment (start 114.54 81.54) (end 114.54 82.38) (width 0.25) (layer B.Cu) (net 10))
 (segment (start 113 80) (end 114.54 81.54) (width 0.25) (layer B.Cu) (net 10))
 (segment (start 111 80) (end 113 80) (width 0.25) (layer B.Cu) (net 10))
 (via (at 111 80) (size 0.762) (drill 0.381) (layers F.Cu B.Cu) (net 10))
 (segment (start 110 80) (end 111 80) (width 0.25) (layer F.Cu) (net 10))
 (segment (start 110 76) (end 110 80) (width 0.25) (layer F.Cu) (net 10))
 (via (at 110 76) (size 0.762) (drill 0.381) (layers F.Cu B.Cu) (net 10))
 (segment (start 113 76) (end 110 76) (width 0.25) (layer B.Cu) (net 10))
 (segment (start 114.46 74.54) (end 113 76) (width 0.25) (layer B.Cu) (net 10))
 (segment (start 121 120) (end 123 120) (width 0.25) (layer B.Cu) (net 10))
 (segment (start 114.54 79.46) (end 114.54 82.38) (width 0.25) (layer B.Cu) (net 10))
 (segment (start 115 79) (end 114.54 79.46) (width 0.25) (layer B.Cu) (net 10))
 (segment (start 125 79) (end 115 79) (width 0.25) (layer B.Cu) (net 10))
 (segment (start 125 118) (end 125 79) (width 0.25) (layer B.Cu) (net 10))
 (segment (start 123 120) (end 125 118) (width 0.25) (layer B.Cu) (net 10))
 (segment (start 119.54 74.54) (end 119.54 74.46) (width 0.25) (layer F.Cu) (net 11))
 (segment (start 119.54 74.46) (end 121 73) (width 0.25) (layer F.Cu) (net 11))
 (segment (start 121 73) (end 121 69) (width 0.25) (layer F.Cu) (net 11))
 (segment (start 121 69) (end 112 69) (width 0.25) (layer F.Cu) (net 11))
 (segment (start 112 69) (end 112 72) (width 0.25) (layer F.Cu) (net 11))
 (segment (start 112 72) (end 110 74) (width 0.25) (layer F.Cu) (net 11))
 (segment (start 110 74) (end 109 74) (width 0.25) (layer F.Cu) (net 11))
 (segment (start 109 74) (end 109 85) (width 0.25) (layer F.Cu) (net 11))
 (segment (start 109 85) (end 110 86) (width 0.25) (layer F.Cu) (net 11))
 (segment (start 110 86) (end 123 86) (width 0.25) (layer F.Cu) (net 11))
 (segment (start 121 104) (end 121 95) (width 0.25) (layer F.Cu) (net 11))
 (segment (start 122.62 82.38) (end 119.62 82.38) (width 0.25) (layer F.Cu) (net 11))
 (segment (start 123 82) (end 122.62 82.38) (width 0.25) (layer F.Cu) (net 11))
 (segment (start 123 95) (end 123 86) (width 0.25) (layer F.Cu) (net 11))
 (segment (start 123 86) (end 123 82) (width 0.25) (layer F.Cu) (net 11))
 (segment (start 121 95) (end 123 95) (width 0.25) (layer F.Cu) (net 11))
 (segment (start 117 77.08) (end 108.92 77.08) (width 0.25) (layer B.Cu) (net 12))
 (segment (start 108 90) (end 112 90) (width 0.25) (layer F.Cu) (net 12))
 (segment (start 108 84) (end 108 90) (width 0.25) (layer F.Cu) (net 12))
 (via (at 108 84) (size 0.762) (drill 0.381) (layers F.Cu B.Cu) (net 12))
 (segment (start 108 78) (end 108 84) (width 0.25) (layer B.Cu) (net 12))
 (segment (start 108.92 77.08) (end 108 78) (width 0.25) (layer B.Cu) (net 12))
 (segment (start 121 127) (end 124 127) (width 0.25) (layer F.Cu) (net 13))
 (segment (start 114.54 92.54) (end 114.54 90) (width 0.25) (layer F.Cu) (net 13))
 (segment (start 115 93) (end 114.54 92.54) (width 0.25) (layer F.Cu) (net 13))
 (segment (start 119 93) (end 115 93) (width 0.25) (layer F.Cu) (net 13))
 (segment (start 119 102) (end 119 93) (width 0.25) (layer F.Cu) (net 13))
 (segment (start 117 102) (end 119 102) (width 0.25) (layer F.Cu) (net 13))
 (segment (start 117 123) (end 117 102) (width 0.25) (layer F.Cu) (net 13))
 (segment (start 116 124) (end 117 123) (width 0.25) (layer F.Cu) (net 13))
 (segment (start 124 124) (end 116 124) (width 0.25) (layer F.Cu) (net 13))
 (segment (start 124 127) (end 124 124) (width 0.25) (layer F.Cu) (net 13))
 (segment (start 121 134) (end 121 132) (width 0.25) (layer B.Cu) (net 14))
 (segment (start 117.08 91.08) (end 117.08 90) (width 0.25) (layer B.Cu) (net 14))
 (segment (start 118 92) (end 117.08 91.08) (width 0.25) (layer B.Cu) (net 14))
 (segment (start 118 130) (end 118 92) (width 0.25) (layer B.Cu) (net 14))
 (segment (start 117 131) (end 118 130) (width 0.25) (layer B.Cu) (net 14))
 (segment (start 120 131) (end 117 131) (width 0.25) (layer B.Cu) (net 14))
 (segment (start 121 132) (end 120 131) (width 0.25) (layer B.Cu) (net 14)))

